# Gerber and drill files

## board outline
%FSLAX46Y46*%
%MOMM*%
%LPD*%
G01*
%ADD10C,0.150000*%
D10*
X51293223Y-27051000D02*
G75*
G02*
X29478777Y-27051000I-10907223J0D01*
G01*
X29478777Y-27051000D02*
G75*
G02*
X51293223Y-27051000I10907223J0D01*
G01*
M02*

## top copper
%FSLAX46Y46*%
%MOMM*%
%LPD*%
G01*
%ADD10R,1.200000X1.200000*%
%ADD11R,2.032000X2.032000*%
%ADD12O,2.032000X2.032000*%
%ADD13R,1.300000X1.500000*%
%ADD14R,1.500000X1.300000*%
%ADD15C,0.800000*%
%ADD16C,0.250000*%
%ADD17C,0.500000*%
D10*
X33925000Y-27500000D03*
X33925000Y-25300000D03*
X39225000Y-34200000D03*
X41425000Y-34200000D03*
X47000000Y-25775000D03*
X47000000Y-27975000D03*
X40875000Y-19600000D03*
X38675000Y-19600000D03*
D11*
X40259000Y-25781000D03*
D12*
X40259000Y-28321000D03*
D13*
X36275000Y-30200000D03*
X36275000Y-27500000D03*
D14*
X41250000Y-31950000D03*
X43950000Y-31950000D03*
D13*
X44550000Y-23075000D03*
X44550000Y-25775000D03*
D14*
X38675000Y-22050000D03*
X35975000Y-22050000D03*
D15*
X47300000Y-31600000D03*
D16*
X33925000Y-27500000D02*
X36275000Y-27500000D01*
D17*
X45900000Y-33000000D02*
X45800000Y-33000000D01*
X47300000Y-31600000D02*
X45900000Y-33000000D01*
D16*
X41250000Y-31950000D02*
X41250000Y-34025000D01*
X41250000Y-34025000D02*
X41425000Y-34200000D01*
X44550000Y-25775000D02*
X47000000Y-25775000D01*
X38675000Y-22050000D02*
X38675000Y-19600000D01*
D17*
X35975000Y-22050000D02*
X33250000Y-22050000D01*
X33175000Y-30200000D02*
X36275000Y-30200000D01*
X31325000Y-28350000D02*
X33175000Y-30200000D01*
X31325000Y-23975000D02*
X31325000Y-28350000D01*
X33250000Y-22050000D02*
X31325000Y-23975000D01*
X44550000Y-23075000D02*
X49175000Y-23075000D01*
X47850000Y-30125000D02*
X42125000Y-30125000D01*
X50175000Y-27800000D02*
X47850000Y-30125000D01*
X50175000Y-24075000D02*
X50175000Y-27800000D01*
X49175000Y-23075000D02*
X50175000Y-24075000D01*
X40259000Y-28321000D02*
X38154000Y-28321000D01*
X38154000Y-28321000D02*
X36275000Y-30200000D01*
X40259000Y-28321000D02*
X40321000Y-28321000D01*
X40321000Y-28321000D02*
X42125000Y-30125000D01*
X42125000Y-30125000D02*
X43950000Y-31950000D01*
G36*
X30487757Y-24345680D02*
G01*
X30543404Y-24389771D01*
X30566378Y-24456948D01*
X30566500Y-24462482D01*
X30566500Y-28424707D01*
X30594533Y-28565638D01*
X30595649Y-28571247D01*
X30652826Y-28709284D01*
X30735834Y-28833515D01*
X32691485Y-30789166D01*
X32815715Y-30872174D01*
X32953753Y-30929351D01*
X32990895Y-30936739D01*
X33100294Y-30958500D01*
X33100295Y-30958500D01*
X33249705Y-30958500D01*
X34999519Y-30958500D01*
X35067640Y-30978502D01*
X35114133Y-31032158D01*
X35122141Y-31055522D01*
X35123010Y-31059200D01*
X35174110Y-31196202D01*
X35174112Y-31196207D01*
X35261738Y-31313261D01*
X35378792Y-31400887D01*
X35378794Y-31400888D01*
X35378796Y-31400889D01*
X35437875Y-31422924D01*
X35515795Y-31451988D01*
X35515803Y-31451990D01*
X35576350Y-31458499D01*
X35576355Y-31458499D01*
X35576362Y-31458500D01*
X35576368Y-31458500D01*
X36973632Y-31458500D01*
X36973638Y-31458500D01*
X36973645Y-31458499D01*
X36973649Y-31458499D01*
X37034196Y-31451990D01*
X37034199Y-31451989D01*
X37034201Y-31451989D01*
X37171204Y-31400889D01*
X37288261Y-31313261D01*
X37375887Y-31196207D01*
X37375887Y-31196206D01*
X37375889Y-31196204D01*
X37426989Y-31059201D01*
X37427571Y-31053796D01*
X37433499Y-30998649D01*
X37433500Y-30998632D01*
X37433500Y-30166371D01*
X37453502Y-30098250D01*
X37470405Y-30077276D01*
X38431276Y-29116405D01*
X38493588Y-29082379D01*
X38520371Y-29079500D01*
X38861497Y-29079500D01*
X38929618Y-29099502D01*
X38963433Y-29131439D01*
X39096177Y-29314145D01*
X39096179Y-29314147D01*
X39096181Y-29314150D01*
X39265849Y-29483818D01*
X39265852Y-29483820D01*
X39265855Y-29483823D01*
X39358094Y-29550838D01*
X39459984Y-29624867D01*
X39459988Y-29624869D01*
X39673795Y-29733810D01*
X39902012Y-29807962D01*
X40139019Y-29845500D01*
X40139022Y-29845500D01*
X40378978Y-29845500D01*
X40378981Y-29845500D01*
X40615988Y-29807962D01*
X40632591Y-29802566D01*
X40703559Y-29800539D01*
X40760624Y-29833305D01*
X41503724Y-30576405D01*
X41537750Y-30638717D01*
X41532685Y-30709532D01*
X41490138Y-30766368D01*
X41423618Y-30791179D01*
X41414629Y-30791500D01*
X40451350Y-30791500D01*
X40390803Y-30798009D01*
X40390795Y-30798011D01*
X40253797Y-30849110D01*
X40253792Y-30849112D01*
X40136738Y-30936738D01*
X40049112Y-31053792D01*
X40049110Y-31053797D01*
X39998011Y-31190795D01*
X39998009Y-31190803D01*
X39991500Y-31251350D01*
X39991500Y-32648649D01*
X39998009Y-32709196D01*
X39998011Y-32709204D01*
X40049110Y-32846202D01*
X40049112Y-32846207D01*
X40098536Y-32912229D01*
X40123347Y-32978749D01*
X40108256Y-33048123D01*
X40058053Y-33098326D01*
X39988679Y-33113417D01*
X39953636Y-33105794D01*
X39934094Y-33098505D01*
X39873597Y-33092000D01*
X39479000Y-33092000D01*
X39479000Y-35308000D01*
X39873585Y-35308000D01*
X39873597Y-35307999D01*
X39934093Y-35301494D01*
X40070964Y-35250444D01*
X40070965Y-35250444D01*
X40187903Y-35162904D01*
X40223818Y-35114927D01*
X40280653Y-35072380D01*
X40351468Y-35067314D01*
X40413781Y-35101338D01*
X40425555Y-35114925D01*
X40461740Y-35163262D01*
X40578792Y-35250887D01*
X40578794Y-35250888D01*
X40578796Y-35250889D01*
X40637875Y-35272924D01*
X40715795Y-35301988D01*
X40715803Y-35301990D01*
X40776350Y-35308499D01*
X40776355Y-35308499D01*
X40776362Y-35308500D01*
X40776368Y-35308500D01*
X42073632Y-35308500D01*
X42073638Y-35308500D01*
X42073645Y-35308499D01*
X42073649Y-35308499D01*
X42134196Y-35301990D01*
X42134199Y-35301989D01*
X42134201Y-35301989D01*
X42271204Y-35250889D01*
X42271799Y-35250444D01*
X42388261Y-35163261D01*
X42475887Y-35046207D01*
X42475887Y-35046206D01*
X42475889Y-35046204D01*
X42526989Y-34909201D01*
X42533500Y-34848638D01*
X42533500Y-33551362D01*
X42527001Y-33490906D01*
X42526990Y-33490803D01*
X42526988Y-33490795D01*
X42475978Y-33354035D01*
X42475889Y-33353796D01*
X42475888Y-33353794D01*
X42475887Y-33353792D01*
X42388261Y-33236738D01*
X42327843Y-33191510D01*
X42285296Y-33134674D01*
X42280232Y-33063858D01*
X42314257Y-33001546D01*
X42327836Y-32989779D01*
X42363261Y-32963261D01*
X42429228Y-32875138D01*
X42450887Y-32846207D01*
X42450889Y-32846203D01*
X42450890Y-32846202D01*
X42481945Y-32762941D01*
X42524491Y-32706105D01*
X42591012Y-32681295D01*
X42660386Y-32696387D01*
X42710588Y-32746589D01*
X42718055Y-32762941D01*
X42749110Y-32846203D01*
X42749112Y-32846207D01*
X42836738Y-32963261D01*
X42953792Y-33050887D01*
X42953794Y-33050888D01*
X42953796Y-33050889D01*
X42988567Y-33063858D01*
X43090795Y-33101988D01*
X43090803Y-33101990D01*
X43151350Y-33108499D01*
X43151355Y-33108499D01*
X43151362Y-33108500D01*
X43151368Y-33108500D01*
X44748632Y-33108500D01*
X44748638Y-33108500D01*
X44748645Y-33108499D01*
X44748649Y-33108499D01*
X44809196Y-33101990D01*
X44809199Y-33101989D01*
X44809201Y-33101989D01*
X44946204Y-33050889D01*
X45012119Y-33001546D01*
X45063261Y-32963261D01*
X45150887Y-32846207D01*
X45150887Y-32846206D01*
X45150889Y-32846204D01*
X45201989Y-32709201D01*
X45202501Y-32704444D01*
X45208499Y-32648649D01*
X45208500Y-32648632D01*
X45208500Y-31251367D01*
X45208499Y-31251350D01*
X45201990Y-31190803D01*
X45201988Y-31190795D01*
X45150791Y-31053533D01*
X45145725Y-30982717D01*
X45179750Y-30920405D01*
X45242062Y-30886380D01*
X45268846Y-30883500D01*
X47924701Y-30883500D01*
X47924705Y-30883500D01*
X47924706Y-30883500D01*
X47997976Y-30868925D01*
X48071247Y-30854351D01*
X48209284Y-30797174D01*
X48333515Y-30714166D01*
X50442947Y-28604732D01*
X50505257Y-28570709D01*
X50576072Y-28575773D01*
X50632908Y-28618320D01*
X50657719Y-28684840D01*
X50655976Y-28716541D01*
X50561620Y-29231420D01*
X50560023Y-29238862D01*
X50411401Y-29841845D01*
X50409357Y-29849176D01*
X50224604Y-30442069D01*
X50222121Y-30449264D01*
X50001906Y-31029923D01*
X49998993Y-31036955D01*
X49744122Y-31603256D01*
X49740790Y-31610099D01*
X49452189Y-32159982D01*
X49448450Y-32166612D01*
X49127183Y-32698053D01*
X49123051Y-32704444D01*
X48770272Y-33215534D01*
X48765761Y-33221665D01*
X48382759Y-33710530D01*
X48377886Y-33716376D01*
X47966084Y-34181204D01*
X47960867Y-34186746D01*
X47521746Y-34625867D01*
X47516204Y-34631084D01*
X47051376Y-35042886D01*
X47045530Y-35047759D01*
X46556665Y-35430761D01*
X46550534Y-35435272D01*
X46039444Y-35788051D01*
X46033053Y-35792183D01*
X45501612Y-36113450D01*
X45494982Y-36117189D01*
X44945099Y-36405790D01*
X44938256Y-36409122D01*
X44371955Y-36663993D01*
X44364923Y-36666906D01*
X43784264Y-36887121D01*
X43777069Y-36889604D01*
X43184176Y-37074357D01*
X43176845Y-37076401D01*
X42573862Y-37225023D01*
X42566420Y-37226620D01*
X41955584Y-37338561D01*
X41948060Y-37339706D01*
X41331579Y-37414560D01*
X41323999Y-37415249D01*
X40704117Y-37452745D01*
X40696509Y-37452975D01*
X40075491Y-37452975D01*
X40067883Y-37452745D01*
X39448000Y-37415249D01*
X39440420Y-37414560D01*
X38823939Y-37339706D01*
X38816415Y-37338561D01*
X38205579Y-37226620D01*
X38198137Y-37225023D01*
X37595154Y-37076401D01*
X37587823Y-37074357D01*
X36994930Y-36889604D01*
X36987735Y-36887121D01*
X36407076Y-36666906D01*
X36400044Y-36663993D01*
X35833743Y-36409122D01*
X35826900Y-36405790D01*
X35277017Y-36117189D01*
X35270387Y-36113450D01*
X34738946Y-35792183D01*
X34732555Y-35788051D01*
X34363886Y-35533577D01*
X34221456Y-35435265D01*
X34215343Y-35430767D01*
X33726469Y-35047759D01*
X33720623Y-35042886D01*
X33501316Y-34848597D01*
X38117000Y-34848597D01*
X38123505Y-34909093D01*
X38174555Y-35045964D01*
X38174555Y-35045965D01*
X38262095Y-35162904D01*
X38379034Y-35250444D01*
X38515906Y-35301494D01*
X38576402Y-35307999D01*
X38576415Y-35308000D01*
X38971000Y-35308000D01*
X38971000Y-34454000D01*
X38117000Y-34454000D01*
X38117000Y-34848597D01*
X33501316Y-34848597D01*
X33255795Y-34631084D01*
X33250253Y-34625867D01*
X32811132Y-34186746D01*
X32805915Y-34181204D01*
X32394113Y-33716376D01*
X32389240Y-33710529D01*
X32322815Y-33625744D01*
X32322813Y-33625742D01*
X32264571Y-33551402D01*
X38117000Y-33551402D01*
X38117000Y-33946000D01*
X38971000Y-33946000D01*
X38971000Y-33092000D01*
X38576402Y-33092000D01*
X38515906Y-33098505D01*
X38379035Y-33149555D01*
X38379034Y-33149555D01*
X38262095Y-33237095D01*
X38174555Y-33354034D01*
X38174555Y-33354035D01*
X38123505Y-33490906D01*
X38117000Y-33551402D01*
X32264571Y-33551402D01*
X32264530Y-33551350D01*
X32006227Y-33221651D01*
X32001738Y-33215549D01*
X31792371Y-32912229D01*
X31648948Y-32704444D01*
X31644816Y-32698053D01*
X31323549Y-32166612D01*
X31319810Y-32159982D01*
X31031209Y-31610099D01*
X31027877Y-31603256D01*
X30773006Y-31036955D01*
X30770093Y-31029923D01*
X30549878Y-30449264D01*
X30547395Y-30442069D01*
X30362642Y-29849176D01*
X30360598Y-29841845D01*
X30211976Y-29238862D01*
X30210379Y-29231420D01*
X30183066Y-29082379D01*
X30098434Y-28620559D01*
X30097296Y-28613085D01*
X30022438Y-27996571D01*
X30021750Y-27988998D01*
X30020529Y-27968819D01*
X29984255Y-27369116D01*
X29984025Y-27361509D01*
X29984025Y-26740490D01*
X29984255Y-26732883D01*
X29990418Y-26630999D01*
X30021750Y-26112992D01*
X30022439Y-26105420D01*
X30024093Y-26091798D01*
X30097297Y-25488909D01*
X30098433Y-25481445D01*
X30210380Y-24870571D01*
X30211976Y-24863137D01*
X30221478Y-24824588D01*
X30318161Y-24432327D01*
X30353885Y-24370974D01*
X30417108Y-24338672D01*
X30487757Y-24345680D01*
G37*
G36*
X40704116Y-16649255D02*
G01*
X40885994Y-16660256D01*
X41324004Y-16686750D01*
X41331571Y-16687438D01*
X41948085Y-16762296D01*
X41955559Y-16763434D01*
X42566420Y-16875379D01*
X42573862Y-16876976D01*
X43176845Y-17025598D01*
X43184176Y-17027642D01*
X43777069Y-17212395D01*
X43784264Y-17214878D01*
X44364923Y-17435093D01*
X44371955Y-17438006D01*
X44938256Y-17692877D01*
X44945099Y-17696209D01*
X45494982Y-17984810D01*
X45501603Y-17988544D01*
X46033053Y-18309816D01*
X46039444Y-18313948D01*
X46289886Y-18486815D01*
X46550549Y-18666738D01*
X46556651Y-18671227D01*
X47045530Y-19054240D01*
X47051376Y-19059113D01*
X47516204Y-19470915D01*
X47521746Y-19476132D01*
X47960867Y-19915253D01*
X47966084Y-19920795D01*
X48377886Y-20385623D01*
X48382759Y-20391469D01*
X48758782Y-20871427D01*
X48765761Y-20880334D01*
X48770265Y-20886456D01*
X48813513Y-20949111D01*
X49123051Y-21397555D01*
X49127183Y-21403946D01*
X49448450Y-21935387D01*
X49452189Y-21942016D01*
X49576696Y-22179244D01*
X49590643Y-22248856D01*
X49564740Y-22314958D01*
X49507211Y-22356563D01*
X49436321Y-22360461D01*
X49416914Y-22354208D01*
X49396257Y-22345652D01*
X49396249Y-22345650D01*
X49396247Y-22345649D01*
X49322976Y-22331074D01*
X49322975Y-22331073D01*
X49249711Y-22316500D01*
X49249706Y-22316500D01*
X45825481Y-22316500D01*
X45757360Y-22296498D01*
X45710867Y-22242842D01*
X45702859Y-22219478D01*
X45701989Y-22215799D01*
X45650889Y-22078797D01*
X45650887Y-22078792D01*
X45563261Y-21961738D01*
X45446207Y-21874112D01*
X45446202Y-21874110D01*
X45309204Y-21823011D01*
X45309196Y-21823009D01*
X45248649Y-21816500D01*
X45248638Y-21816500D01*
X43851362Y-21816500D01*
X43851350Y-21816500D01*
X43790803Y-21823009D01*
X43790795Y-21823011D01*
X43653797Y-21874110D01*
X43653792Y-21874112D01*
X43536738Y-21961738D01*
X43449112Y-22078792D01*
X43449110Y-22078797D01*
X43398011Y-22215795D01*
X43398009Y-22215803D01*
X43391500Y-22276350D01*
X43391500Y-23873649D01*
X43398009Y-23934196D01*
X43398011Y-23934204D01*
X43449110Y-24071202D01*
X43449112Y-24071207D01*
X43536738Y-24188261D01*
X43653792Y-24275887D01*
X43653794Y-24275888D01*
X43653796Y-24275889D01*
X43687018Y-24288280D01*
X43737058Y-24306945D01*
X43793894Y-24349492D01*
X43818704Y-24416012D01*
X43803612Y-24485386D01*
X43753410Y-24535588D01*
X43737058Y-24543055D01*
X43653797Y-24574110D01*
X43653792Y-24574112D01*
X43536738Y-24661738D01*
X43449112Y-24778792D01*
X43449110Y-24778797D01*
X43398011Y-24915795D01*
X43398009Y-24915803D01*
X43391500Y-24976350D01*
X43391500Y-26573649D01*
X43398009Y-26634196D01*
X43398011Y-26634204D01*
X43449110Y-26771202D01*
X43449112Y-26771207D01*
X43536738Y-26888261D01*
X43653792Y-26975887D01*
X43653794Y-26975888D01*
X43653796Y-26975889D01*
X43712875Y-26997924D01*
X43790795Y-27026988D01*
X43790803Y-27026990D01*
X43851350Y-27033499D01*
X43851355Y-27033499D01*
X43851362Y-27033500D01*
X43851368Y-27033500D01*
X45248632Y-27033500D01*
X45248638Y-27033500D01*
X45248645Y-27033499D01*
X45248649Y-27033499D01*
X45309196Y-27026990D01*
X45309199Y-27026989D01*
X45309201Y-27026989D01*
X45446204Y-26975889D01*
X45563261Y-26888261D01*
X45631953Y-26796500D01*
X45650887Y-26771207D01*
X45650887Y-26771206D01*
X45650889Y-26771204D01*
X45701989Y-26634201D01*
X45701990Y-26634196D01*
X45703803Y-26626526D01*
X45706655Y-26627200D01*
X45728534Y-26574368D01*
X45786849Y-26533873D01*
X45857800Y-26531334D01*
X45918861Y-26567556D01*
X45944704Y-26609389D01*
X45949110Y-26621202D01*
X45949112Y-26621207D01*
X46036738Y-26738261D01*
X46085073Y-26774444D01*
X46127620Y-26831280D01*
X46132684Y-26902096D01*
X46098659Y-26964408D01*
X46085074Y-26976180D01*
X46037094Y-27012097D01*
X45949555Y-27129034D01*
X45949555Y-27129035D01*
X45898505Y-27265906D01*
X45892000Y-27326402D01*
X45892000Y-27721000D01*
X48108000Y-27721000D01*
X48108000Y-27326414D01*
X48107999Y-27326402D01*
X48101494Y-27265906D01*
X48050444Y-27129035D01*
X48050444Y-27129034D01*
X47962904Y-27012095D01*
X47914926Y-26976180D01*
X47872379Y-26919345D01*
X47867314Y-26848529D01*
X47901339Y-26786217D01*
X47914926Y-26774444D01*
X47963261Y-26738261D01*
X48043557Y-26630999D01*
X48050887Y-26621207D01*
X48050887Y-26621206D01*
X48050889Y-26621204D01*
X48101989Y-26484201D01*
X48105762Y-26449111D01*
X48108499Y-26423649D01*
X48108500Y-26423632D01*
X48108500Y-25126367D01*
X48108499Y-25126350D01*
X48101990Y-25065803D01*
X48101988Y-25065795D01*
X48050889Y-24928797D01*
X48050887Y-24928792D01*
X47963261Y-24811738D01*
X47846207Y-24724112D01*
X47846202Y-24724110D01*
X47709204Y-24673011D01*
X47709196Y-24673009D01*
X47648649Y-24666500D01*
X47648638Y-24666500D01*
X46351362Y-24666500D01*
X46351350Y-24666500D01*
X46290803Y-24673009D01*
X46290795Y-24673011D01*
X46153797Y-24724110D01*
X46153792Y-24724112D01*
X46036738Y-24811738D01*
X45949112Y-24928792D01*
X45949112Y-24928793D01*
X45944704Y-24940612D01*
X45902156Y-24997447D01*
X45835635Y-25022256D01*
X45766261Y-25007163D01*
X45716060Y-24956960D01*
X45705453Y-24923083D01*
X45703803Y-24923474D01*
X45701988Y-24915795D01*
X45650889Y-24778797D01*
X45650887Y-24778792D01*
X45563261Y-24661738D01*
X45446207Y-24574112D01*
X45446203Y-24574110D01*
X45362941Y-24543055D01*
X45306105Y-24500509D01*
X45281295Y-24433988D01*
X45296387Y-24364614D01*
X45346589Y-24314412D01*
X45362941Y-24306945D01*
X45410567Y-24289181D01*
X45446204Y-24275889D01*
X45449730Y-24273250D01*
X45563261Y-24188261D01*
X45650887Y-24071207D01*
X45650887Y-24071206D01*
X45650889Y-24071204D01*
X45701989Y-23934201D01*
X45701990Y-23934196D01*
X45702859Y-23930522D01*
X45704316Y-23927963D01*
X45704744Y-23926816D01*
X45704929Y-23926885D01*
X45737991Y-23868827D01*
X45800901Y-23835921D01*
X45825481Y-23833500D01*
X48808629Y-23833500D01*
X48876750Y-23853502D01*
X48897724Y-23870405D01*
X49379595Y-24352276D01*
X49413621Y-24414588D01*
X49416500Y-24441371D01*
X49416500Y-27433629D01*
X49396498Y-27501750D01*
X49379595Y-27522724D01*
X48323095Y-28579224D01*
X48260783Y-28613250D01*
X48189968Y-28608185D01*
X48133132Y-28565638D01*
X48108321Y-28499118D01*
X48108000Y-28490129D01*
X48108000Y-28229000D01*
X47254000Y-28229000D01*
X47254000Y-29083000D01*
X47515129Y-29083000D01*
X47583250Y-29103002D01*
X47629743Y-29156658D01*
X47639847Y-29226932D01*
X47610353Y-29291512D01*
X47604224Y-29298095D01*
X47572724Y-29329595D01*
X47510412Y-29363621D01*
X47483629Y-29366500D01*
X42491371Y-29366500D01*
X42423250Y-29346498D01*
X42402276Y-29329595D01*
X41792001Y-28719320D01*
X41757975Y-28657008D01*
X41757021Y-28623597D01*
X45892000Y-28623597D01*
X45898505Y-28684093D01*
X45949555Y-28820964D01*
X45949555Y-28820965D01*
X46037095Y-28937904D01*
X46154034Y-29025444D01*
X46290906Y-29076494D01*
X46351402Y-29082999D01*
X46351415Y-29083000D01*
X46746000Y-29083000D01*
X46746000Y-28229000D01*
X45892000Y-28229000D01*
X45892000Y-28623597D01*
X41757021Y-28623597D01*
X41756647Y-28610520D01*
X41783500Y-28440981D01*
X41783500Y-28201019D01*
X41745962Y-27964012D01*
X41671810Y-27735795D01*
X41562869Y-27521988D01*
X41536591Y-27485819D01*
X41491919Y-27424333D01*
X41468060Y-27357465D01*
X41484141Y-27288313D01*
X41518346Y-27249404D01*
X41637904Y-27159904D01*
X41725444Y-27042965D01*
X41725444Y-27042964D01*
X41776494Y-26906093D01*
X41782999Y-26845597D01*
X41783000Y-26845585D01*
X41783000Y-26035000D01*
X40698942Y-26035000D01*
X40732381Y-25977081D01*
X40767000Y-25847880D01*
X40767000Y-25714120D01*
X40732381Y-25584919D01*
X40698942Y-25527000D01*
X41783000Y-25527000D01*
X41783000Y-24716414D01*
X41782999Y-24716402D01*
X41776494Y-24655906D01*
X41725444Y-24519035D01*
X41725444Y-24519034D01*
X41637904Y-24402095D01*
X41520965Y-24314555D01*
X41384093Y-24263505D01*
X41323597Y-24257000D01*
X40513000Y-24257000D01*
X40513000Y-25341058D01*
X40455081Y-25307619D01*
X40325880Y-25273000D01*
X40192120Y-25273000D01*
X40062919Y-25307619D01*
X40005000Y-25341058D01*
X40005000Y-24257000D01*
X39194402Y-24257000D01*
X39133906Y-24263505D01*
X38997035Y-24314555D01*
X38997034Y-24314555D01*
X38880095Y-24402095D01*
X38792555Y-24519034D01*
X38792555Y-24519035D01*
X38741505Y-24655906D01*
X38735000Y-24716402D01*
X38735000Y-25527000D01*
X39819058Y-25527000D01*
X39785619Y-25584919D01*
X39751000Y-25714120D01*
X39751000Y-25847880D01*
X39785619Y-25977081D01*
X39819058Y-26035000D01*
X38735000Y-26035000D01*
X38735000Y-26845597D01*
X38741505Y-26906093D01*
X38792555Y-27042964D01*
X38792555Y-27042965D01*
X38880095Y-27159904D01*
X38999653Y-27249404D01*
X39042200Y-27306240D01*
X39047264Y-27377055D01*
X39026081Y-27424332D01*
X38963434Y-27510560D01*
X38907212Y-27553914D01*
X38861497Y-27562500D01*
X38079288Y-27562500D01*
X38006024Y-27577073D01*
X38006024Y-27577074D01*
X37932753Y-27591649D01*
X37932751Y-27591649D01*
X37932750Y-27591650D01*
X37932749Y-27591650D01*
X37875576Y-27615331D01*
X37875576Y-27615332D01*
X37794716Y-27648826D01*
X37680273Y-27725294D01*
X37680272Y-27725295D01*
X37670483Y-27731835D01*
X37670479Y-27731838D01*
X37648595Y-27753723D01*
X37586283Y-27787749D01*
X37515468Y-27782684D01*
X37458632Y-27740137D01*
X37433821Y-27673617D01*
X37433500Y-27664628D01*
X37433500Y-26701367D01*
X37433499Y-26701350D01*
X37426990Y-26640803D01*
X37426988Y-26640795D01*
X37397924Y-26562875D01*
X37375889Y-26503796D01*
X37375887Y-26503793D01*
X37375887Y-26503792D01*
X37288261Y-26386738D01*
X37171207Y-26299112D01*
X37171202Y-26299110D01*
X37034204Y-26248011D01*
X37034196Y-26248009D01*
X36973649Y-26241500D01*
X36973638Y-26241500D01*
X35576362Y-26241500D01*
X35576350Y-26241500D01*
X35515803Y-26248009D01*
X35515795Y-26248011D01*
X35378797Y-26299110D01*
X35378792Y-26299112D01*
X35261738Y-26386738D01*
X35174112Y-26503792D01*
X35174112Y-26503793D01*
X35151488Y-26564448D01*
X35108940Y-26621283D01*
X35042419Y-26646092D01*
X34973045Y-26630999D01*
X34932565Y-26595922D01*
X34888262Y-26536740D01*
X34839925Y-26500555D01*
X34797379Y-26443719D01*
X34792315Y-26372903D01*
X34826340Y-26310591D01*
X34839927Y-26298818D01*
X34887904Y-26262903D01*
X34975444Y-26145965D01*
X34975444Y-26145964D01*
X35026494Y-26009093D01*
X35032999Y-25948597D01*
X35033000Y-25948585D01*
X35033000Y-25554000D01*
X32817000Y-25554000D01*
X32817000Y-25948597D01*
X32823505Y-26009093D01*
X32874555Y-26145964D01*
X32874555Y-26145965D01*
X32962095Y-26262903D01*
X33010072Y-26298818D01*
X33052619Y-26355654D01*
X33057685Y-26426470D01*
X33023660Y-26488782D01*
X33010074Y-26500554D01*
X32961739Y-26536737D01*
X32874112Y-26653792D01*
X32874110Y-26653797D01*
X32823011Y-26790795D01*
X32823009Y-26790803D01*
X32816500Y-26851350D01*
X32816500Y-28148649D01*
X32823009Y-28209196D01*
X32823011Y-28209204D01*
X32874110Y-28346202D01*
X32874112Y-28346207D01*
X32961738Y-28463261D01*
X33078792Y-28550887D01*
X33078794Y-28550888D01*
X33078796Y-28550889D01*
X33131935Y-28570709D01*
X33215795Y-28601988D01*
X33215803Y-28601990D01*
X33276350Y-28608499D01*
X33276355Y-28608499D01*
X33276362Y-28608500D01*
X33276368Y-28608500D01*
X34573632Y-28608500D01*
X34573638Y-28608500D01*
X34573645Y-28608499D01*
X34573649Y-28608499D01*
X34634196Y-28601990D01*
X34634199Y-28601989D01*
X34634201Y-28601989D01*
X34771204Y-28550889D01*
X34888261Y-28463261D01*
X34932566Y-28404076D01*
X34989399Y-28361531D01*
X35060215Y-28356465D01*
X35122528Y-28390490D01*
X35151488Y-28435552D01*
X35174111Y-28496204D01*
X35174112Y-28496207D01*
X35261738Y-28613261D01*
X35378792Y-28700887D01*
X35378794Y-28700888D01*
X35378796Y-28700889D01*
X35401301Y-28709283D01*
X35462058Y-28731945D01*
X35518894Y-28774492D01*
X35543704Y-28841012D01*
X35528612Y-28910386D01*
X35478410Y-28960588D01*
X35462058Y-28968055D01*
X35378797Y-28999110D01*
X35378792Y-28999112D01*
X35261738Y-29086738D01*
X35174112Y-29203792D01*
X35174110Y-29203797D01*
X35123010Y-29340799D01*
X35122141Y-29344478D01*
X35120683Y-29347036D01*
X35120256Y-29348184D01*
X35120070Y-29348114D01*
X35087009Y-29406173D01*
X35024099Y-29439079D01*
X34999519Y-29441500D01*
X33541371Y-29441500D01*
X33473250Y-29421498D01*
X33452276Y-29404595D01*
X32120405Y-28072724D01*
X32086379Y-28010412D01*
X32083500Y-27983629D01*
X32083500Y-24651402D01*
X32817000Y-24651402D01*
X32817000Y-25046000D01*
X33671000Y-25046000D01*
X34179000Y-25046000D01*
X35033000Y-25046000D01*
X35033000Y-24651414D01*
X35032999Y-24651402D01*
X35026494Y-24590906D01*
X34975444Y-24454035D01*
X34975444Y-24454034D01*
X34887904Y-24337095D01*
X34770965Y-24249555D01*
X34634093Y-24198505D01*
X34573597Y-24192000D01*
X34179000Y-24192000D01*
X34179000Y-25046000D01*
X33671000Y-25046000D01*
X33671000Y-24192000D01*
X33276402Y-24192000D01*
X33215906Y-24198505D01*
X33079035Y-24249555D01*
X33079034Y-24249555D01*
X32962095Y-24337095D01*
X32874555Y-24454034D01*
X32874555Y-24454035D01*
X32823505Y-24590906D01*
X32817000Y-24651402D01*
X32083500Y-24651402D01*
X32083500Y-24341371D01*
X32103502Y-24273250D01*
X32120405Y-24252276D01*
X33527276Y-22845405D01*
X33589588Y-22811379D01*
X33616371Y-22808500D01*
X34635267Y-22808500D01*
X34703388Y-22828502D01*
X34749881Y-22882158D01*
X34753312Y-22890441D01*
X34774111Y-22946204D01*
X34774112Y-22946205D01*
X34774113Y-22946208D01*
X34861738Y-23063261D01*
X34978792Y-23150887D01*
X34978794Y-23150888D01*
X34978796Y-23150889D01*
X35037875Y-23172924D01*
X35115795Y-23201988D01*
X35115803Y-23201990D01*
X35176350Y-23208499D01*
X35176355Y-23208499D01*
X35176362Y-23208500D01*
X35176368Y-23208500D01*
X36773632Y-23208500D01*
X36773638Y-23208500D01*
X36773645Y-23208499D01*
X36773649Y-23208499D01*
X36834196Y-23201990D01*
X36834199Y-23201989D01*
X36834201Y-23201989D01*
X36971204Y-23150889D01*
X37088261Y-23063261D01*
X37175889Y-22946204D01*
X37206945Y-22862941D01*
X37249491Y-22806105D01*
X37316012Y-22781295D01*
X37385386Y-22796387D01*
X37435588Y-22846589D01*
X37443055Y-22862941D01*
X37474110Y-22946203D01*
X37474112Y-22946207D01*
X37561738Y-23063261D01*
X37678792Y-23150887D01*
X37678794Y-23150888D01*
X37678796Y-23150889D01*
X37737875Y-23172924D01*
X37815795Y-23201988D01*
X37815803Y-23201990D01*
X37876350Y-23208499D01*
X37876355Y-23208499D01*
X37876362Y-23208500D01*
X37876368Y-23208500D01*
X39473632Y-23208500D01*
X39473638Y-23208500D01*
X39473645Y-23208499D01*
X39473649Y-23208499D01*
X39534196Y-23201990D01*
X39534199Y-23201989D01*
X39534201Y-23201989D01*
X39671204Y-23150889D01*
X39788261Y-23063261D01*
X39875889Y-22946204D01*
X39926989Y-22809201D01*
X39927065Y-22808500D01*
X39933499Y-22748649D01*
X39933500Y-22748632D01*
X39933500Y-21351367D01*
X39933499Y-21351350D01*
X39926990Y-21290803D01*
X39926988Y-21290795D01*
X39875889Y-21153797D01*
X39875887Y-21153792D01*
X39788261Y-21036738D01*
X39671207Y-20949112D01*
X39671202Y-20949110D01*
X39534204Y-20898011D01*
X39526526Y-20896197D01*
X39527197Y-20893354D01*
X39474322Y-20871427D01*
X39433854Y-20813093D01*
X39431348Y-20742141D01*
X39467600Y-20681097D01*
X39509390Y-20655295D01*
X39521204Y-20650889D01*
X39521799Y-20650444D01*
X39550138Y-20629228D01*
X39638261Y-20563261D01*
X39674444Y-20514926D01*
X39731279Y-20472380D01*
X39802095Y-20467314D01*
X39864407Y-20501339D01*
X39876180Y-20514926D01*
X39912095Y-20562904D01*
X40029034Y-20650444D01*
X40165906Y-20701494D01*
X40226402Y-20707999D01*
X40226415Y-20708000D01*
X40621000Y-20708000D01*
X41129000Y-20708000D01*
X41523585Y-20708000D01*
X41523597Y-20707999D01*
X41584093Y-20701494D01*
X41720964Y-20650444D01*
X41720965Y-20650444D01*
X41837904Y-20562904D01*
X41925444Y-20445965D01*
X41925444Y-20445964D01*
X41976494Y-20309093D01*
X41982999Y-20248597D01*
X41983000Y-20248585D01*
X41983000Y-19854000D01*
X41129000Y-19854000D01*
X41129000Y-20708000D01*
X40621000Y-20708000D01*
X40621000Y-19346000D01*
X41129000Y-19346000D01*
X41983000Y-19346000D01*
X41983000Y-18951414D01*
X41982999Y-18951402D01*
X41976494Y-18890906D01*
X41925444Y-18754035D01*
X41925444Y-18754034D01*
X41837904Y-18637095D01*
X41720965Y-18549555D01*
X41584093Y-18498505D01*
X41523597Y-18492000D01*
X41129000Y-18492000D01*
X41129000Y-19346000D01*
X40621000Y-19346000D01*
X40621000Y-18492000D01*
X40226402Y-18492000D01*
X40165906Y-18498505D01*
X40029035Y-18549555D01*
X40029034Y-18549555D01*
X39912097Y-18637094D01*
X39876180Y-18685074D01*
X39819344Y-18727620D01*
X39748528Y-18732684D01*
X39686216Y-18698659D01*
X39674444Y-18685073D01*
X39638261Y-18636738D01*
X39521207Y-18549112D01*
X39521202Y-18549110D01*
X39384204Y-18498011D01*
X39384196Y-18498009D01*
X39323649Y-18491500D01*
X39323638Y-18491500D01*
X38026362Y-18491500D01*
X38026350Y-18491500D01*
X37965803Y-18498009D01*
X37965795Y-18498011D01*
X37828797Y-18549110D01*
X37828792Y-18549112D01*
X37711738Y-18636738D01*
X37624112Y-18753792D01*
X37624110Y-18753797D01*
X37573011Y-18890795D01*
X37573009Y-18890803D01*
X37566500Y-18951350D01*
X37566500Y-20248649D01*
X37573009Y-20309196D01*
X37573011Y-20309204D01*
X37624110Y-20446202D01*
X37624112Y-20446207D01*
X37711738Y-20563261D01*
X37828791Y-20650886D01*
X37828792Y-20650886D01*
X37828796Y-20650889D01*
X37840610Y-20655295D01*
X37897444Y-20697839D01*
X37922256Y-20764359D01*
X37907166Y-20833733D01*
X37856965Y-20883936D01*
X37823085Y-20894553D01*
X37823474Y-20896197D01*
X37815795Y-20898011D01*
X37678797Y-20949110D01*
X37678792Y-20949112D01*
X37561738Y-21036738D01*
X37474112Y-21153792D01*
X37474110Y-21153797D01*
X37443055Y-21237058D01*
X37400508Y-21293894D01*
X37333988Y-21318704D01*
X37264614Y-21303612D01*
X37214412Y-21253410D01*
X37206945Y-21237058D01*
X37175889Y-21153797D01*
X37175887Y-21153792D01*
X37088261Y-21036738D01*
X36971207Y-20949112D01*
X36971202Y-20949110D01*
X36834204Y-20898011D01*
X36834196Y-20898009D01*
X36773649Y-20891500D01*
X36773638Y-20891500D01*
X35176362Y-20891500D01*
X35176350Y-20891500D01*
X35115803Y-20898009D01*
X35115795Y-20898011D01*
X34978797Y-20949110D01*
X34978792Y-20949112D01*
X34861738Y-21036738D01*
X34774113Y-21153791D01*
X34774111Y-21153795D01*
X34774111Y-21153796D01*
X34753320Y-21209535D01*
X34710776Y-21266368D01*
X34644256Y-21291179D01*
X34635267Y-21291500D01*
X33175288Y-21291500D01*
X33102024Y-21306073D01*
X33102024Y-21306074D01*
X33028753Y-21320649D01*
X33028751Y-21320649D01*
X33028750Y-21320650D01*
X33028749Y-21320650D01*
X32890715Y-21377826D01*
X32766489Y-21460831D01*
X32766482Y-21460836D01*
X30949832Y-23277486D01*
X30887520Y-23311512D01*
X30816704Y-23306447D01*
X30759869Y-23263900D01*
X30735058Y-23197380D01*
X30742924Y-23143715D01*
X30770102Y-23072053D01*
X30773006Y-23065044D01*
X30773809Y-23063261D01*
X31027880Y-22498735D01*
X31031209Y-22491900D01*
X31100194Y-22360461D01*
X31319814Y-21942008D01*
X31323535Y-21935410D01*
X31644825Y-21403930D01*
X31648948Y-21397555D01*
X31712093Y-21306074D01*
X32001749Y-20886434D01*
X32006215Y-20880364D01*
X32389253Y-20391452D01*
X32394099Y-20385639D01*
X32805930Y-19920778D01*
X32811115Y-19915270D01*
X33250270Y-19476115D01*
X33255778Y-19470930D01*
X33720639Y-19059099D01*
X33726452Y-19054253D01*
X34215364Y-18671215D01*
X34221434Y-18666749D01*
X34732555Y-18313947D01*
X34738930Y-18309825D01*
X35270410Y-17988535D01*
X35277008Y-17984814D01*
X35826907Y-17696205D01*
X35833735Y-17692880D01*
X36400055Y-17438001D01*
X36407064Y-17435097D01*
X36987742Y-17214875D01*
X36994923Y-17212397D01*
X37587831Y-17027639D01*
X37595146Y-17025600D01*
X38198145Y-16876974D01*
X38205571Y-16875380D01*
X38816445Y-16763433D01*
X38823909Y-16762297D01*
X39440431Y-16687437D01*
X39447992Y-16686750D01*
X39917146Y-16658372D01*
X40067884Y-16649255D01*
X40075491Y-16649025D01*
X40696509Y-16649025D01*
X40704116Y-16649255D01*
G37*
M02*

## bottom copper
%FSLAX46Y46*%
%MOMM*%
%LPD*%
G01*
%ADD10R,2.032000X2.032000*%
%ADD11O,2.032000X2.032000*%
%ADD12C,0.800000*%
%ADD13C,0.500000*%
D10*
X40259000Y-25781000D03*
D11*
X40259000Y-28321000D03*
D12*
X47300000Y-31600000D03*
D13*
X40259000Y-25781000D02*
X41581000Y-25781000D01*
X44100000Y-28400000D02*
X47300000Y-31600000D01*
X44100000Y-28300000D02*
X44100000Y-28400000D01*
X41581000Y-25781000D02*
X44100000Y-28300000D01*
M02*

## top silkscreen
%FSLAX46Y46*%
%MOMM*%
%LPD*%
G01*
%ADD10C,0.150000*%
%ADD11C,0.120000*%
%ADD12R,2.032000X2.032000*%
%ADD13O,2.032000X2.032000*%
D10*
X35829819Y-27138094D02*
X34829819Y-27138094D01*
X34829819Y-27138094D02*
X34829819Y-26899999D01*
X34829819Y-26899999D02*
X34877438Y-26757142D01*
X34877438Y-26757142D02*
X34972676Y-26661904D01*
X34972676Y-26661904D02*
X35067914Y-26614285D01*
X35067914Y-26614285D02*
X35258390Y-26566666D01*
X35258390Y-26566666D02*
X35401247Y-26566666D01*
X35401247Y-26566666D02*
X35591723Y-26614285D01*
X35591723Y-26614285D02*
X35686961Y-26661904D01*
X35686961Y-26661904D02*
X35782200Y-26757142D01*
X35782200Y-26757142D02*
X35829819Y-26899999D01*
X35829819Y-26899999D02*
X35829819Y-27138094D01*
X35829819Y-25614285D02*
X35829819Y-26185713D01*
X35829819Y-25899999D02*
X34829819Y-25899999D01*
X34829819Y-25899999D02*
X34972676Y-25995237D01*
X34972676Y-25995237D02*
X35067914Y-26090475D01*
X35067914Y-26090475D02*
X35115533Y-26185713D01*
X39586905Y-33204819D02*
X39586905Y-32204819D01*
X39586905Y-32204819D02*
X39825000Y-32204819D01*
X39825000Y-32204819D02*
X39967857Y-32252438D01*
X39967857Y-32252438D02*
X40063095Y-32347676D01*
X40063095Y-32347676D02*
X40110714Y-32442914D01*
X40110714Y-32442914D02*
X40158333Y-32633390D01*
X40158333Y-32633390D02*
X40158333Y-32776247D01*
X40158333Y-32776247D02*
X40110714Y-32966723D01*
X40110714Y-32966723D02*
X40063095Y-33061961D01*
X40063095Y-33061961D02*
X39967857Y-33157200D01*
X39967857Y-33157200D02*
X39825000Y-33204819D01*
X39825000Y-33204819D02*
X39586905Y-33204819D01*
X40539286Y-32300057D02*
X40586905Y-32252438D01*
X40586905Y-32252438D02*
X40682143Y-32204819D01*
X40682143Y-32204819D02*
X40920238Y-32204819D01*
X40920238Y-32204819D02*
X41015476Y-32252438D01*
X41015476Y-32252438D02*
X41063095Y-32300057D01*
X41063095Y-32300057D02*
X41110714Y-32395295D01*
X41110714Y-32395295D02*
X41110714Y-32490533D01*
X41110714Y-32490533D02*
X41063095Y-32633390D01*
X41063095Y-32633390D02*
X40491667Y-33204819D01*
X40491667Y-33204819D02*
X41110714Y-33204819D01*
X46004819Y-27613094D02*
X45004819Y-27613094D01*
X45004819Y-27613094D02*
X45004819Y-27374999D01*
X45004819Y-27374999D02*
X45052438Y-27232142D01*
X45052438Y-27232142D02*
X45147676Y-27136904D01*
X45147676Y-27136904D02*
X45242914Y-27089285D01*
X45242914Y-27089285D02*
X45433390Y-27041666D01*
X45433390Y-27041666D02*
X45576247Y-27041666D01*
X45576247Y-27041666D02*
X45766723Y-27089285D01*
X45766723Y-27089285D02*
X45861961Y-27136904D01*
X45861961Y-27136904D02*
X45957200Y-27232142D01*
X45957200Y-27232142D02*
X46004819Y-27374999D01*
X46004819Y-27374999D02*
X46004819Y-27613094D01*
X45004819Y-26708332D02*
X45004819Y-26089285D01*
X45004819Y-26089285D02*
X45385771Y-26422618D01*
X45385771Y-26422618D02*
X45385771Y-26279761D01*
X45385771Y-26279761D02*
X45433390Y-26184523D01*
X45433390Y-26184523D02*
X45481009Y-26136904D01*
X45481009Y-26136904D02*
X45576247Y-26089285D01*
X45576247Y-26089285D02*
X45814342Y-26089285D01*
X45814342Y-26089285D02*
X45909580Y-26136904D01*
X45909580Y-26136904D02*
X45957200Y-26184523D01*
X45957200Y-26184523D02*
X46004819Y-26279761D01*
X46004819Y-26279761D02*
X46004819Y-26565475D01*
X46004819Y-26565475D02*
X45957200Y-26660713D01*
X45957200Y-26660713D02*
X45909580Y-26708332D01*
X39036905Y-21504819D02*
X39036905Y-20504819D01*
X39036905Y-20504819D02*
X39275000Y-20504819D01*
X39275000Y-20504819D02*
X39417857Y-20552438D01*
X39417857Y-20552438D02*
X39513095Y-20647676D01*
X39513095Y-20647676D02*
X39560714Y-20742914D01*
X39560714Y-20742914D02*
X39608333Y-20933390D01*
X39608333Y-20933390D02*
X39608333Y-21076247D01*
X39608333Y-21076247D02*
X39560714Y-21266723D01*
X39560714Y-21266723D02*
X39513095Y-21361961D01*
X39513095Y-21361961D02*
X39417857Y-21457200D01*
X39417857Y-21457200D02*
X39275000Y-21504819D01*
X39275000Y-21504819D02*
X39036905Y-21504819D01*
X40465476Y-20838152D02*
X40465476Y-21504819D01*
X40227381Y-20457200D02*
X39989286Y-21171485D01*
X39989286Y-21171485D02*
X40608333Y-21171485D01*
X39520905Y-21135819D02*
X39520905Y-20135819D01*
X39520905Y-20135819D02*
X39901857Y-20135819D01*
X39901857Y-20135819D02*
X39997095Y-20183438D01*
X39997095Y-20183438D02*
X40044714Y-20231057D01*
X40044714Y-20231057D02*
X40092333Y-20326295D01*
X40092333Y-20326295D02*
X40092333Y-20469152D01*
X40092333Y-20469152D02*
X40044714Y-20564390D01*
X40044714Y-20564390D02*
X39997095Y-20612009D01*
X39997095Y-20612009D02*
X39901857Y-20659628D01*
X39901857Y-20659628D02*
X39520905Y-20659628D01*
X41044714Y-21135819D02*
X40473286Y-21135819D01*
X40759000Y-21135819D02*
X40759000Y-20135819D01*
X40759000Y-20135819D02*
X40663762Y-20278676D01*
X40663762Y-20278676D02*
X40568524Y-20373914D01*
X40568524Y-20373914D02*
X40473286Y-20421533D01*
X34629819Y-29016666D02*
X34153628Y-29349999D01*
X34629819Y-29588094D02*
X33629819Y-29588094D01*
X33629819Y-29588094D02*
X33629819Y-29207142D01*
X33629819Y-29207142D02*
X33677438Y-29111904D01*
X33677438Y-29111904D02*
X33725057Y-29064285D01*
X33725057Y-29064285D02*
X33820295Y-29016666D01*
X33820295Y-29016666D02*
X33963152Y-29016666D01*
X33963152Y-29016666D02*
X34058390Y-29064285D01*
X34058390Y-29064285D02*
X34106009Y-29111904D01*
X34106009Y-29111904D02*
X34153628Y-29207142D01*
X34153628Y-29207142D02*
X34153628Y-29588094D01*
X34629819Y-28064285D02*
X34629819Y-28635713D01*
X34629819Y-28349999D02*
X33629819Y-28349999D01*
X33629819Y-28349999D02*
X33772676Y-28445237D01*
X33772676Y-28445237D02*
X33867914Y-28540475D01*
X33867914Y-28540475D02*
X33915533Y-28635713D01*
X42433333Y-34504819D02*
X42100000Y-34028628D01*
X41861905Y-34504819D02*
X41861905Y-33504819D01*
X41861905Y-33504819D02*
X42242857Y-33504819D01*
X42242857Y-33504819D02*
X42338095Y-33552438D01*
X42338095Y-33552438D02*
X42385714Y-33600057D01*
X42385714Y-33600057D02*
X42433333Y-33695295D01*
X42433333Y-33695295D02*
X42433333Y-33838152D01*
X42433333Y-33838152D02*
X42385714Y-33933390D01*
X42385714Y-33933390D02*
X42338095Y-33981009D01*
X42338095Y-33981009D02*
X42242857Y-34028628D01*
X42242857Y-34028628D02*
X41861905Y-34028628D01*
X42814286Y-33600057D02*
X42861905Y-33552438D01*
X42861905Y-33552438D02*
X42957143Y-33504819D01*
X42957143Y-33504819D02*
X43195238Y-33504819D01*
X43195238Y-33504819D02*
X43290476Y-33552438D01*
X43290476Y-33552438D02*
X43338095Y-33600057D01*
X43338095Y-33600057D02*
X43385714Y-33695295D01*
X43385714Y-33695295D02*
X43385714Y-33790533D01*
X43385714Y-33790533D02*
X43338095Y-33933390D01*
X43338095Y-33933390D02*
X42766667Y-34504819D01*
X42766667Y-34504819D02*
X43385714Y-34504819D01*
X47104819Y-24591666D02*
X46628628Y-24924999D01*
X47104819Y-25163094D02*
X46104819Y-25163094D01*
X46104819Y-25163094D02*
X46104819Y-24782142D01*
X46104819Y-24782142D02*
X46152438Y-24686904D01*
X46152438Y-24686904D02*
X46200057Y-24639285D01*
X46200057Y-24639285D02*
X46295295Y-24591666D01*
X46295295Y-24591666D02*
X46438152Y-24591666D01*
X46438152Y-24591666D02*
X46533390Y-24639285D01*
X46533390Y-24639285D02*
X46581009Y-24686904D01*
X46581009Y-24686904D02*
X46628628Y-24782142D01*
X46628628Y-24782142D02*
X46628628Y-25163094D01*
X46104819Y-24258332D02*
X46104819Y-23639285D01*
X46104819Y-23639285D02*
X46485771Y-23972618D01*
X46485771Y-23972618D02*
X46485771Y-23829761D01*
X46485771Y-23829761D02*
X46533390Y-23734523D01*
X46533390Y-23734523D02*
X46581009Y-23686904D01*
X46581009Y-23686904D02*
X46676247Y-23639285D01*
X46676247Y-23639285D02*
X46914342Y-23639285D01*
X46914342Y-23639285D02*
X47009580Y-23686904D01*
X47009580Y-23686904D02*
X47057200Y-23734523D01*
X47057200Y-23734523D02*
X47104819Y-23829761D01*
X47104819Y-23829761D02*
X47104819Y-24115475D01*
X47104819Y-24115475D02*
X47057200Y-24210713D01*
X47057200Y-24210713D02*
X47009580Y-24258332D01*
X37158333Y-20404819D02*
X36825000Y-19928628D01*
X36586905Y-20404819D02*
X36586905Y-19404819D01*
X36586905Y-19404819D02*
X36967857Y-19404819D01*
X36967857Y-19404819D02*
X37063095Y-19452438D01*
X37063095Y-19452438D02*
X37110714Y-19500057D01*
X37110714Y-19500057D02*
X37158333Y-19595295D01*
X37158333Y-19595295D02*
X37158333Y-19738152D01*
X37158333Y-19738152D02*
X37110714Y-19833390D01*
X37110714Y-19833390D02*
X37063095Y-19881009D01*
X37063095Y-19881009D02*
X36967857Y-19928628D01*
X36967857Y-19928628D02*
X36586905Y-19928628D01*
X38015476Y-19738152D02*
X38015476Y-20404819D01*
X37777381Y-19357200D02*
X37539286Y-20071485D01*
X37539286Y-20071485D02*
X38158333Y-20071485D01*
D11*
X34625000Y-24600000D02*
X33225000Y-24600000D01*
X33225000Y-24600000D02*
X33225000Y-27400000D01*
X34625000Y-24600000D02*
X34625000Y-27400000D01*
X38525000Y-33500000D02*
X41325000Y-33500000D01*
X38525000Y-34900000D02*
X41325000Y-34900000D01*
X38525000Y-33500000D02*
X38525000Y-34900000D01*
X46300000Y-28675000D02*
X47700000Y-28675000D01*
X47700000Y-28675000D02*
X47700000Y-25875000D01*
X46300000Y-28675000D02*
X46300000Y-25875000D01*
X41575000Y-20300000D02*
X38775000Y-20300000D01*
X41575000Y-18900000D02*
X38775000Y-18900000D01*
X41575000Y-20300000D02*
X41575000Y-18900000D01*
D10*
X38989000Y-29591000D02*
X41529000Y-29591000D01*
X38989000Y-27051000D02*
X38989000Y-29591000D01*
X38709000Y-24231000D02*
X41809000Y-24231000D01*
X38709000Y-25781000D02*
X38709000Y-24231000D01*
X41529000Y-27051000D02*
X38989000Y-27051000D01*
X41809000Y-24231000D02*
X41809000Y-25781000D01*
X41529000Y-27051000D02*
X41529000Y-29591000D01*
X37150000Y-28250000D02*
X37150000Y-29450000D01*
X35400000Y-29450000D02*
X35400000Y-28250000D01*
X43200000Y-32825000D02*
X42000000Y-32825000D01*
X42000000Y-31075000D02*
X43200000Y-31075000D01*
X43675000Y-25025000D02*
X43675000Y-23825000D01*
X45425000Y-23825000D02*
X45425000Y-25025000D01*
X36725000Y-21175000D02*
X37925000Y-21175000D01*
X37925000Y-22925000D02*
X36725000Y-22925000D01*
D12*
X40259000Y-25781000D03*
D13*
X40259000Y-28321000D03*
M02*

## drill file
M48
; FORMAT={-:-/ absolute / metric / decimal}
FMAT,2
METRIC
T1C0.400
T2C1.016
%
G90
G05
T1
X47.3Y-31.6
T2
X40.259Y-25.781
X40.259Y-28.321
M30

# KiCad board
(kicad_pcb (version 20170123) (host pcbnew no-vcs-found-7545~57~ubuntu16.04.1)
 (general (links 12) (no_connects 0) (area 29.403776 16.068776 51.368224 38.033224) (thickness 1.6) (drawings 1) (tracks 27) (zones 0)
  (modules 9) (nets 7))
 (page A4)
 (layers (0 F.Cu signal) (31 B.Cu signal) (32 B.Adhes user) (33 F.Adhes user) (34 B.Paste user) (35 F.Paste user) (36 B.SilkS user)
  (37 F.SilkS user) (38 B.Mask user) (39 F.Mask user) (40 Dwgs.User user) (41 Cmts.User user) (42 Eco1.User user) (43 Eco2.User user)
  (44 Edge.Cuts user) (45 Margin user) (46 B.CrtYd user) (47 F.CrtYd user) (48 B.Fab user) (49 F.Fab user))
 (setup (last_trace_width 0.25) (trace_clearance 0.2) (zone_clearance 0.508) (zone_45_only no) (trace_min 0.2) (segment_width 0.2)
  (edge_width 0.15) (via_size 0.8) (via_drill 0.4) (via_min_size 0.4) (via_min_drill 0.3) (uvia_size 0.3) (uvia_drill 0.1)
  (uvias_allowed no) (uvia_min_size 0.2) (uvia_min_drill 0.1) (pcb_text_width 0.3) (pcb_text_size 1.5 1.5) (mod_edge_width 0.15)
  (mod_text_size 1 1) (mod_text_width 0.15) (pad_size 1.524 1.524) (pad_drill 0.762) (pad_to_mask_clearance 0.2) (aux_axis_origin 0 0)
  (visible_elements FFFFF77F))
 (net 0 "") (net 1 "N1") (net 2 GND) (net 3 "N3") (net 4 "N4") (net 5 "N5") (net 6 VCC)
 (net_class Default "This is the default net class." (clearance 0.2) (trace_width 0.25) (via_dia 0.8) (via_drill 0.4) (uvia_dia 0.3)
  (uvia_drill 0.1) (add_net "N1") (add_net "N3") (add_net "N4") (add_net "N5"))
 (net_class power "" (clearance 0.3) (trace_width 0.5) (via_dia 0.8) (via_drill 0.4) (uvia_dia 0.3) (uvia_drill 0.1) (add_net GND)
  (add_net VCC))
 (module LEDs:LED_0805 (layer F.Cu) (at 33.925 26.4 270)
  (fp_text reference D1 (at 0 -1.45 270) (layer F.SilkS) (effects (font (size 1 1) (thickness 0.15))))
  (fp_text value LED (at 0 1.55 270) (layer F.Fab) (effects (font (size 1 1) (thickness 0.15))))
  (fp_line (start -1.8 -0.7) (end -1.8 0.7) (layer F.SilkS) (width 0.12))
  (fp_line (start -1.8 0.7) (end 1 0.7) (layer F.SilkS) (width 0.12))
  (fp_line (start -1.8 -0.7) (end 1 -0.7) (layer F.SilkS) (width 0.12))
  (pad 2 smd rect (at 1.1 0 90) (size 1.2 1.2) (layers F.Cu F.Paste F.Mask) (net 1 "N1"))
  (pad 1 smd rect (at -1.1 0 90) (size 1.2 1.2) (layers F.Cu F.Paste F.Mask) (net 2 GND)))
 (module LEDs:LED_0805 (layer F.Cu) (at 40.325 34.2)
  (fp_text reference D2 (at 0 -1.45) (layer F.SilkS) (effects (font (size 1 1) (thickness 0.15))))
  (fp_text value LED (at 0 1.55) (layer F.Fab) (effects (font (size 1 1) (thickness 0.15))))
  (fp_line (start -1.8 -0.7) (end 1 -0.7) (layer F.SilkS) (width 0.12))
  (fp_line (start -1.8 0.7) (end 1 0.7) (layer F.SilkS) (width 0.12))
  (fp_line (start -1.8 -0.7) (end -1.8 0.7) (layer F.SilkS) (width 0.12))
  (pad 1 smd rect (at -1.1 0 180) (size 1.2 1.2) (layers F.Cu F.Paste F.Mask) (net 2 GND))
  (pad 2 smd rect (at 1.1 0 180) (size 1.2 1.2) (layers F.Cu F.Paste F.Mask) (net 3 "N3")))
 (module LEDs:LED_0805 (layer F.Cu) (at 47 26.875 90)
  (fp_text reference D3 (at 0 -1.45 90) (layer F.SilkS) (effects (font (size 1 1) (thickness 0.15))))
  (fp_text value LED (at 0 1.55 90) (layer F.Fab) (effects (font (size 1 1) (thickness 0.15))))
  (fp_line (start -1.8 -0.7) (end -1.8 0.7) (layer F.SilkS) (width 0.12))
  (fp_line (start -1.8 0.7) (end 1 0.7) (layer F.SilkS) (width 0.12))
  (fp_line (start -1.8 -0.7) (end 1 -0.7) (layer F.SilkS) (width 0.12))
  (pad 2 smd rect (at 1.1 0 270) (size 1.2 1.2) (layers F.Cu F.Paste F.Mask) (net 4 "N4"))
  (pad 1 smd rect (at -1.1 0 270) (size 1.2 1.2) (layers F.Cu F.Paste F.Mask) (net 2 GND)))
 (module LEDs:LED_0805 (layer F.Cu) (at 39.775 19.6 180)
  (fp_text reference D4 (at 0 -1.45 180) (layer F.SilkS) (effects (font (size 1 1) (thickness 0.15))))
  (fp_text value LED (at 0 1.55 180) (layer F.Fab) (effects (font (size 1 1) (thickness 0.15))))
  (fp_line (start -1.8 -0.7) (end 1 -0.7) (layer F.SilkS) (width 0.12))
  (fp_line (start -1.8 0.7) (end 1 0.7) (layer F.SilkS) (width 0.12))
  (fp_line (start -1.8 -0.7) (end -1.8 0.7) (layer F.SilkS) (width 0.12))
  (pad 1 smd rect (at -1.1 0) (size 1.2 1.2) (layers F.Cu F.Paste F.Mask) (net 2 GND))
  (pad 2 smd rect (at 1.1 0) (size 1.2 1.2) (layers F.Cu F.Paste F.Mask) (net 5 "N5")))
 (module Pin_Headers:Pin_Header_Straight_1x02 (layer F.Cu) (at 40.259 25.781)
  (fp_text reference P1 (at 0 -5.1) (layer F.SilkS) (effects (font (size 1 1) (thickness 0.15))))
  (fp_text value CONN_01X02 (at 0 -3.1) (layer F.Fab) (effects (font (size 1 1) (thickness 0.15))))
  (fp_line (start -1.27 3.81) (end 1.27 3.81) (layer F.SilkS) (width 0.15))
  (fp_line (start -1.27 1.27) (end -1.27 3.81) (layer F.SilkS) (width 0.15))
  (fp_line (start -1.55 -1.55) (end 1.55 -1.55) (layer F.SilkS) (width 0.15))
  (fp_line (start -1.55 0) (end -1.55 -1.55) (layer F.SilkS) (width 0.15))
  (fp_line (start 1.27 1.27) (end -1.27 1.27) (layer F.SilkS) (width 0.15))
  (fp_line (start 1.55 -1.55) (end 1.55 0) (layer F.SilkS) (width 0.15))
  (fp_line (start 1.27 1.27) (end 1.27 3.81) (layer F.SilkS) (width 0.15))
  (pad 1 thru_hole rect (at 0 0) (size 2.032 2.032) (drill 1.016) (layers *.Cu *.Mask F.SilkS) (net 2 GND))
  (pad 2 thru_hole oval (at 0 2.54) (size 2.032 2.032) (drill 1.016) (layers *.Cu *.Mask F.SilkS) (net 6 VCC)))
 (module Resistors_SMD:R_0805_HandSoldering (layer F.Cu) (at 36.275 28.85 90)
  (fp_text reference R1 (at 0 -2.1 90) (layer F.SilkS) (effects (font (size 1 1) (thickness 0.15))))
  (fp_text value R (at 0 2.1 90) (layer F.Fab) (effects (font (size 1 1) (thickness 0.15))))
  (fp_line (start 0.6 0.875) (end -0.6 0.875) (layer F.SilkS) (width 0.15))
  (fp_line (start -0.6 -0.875) (end 0.6 -0.875) (layer F.SilkS) (width 0.15))
  (pad 1 smd rect (at -1.35 0 90) (size 1.5 1.3) (layers F.Cu F.Paste F.Mask) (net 6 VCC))
  (pad 2 smd rect (at 1.35 0 90) (size 1.5 1.3) (layers F.Cu F.Paste F.Mask) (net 1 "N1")))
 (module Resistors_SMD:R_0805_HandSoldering (layer F.Cu) (at 42.6 31.95 180)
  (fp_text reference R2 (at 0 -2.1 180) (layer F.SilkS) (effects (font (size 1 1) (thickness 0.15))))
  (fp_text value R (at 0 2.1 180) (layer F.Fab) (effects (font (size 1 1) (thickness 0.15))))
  (fp_line (start -0.6 -0.875) (end 0.6 -0.875) (layer F.SilkS) (width 0.15))
  (fp_line (start 0.6 0.875) (end -0.6 0.875) (layer F.SilkS) (width 0.15))
  (pad 2 smd rect (at 1.35 0 180) (size 1.5 1.3) (layers F.Cu F.Paste F.Mask) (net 3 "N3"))
  (pad 1 smd rect (at -1.35 0 180) (size 1.5 1.3) (layers F.Cu F.Paste F.Mask) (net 6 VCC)))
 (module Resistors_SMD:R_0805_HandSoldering (layer F.Cu) (at 44.55 24.425 270)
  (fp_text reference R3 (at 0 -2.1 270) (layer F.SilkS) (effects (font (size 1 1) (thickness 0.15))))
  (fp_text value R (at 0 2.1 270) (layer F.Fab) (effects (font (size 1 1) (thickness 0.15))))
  (fp_line (start 0.6 0.875) (end -0.6 0.875) (layer F.SilkS) (width 0.15))
  (fp_line (start -0.6 -0.875) (end 0.6 -0.875) (layer F.SilkS) (width 0.15))
  (pad 1 smd rect (at -1.35 0 270) (size 1.5 1.3) (layers F.Cu F.Paste F.Mask) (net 6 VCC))
  (pad 2 smd rect (at 1.35 0 270) (size 1.5 1.3) (layers F.Cu F.Paste F.Mask) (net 4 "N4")))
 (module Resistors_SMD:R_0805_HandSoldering (layer F.Cu) (at 37.325 22.05)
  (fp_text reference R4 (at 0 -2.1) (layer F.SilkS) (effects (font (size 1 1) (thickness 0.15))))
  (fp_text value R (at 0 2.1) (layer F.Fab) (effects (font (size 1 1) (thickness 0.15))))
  (fp_line (start -0.6 -0.875) (end 0.6 -0.875) (layer F.SilkS) (width 0.15))
  (fp_line (start 0.6 0.875) (end -0.6 0.875) (layer F.SilkS) (width 0.15))
  (pad 2 smd rect (at 1.35 0) (size 1.5 1.3) (layers F.Cu F.Paste F.Mask) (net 5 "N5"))
  (pad 1 smd rect (at -1.35 0) (size 1.5 1.3) (layers F.Cu F.Paste F.Mask) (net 6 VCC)))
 (gr_circle (center 40.386 27.051) (end 35.306 17.399) (layer Edge.Cuts) (width 0.15))
 (segment (start 33.925 27.5) (end 36.275 27.5) (width 0.25) (layer F.Cu) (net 1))
 (segment (start 40.259 25.781) (end 41.581 25.781) (width 0.5) (layer B.Cu) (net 2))
 (segment (start 45.9 33) (end 45.8 33) (width 0.5) (layer F.Cu) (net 2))
 (segment (start 47.3 31.6) (end 45.9 33) (width 0.5) (layer F.Cu) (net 2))
 (via (at 47.3 31.6) (size 0.8) (drill 0.4) (layers F.Cu B.Cu) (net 2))
 (segment (start 44.1 28.4) (end 47.3 31.6) (width 0.5) (layer B.Cu) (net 2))
 (segment (start 44.1 28.3) (end 44.1 28.4) (width 0.5) (layer B.Cu) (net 2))
 (segment (start 41.581 25.781) (end 44.1 28.3) (width 0.5) (layer B.Cu) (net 2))
 (segment (start 41.25 31.95) (end 41.25 34.025) (width 0.25) (layer F.Cu) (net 3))
 (segment (start 41.25 34.025) (end 41.425 34.2) (width 0.25) (layer F.Cu) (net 3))
 (segment (start 44.55 25.775) (end 47 25.775) (width 0.25) (layer F.Cu) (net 4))
 (segment (start 38.675 22.05) (end 38.675 19.6) (width 0.25) (layer F.Cu) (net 5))
 (segment (start 35.975 22.05) (end 33.25 22.05) (width 0.5) (layer F.Cu) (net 6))
 (segment (start 33.175 30.2) (end 36.275 30.2) (width 0.5) (layer F.Cu) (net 6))
 (segment (start 31.325 28.35) (end 33.175 30.2) (width 0.5) (layer F.Cu) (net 6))
 (segment (start 31.325 23.975) (end 31.325 28.35) (width 0.5) (layer F.Cu) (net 6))
 (segment (start 33.25 22.05) (end 31.325 23.975) (width 0.5) (layer F.Cu) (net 6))
 (segment (start 44.55 23.075) (end 49.175 23.075) (width 0.5) (layer F.Cu) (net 6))
 (segment (start 47.85 30.125) (end 42.125 30.125) (width 0.5) (layer F.Cu) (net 6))
 (segment (start 50.175 27.8) (end 47.85 30.125) (width 0.5) (layer F.Cu) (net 6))
 (segment (start 50.175 24.075) (end 50.175 27.8) (width 0.5) (layer F.Cu) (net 6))
 (segment (start 49.175 23.075) (end 50.175 24.075) (width 0.5) (layer F.Cu) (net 6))
 (segment (start 40.259 28.321) (end 38.154 28.321) (width 0.5) (layer F.Cu) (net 6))
 (segment (start 38.154 28.321) (end 36.275 30.2) (width 0.5) (layer F.Cu) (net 6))
 (segment (start 40.259 28.321) (end 40.321 28.321) (width 0.5) (layer F.Cu) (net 6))
 (segment (start 40.321 28.321) (end 42.125 30.125) (width 0.5) (layer F.Cu) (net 6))
 (segment (start 42.125 30.125) (end 43.95 31.95) (width 0.5) (layer F.Cu) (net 6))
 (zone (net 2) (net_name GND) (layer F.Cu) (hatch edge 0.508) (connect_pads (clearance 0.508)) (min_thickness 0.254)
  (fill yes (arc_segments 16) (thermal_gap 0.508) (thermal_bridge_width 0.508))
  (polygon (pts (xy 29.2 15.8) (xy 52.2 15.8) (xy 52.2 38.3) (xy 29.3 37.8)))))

